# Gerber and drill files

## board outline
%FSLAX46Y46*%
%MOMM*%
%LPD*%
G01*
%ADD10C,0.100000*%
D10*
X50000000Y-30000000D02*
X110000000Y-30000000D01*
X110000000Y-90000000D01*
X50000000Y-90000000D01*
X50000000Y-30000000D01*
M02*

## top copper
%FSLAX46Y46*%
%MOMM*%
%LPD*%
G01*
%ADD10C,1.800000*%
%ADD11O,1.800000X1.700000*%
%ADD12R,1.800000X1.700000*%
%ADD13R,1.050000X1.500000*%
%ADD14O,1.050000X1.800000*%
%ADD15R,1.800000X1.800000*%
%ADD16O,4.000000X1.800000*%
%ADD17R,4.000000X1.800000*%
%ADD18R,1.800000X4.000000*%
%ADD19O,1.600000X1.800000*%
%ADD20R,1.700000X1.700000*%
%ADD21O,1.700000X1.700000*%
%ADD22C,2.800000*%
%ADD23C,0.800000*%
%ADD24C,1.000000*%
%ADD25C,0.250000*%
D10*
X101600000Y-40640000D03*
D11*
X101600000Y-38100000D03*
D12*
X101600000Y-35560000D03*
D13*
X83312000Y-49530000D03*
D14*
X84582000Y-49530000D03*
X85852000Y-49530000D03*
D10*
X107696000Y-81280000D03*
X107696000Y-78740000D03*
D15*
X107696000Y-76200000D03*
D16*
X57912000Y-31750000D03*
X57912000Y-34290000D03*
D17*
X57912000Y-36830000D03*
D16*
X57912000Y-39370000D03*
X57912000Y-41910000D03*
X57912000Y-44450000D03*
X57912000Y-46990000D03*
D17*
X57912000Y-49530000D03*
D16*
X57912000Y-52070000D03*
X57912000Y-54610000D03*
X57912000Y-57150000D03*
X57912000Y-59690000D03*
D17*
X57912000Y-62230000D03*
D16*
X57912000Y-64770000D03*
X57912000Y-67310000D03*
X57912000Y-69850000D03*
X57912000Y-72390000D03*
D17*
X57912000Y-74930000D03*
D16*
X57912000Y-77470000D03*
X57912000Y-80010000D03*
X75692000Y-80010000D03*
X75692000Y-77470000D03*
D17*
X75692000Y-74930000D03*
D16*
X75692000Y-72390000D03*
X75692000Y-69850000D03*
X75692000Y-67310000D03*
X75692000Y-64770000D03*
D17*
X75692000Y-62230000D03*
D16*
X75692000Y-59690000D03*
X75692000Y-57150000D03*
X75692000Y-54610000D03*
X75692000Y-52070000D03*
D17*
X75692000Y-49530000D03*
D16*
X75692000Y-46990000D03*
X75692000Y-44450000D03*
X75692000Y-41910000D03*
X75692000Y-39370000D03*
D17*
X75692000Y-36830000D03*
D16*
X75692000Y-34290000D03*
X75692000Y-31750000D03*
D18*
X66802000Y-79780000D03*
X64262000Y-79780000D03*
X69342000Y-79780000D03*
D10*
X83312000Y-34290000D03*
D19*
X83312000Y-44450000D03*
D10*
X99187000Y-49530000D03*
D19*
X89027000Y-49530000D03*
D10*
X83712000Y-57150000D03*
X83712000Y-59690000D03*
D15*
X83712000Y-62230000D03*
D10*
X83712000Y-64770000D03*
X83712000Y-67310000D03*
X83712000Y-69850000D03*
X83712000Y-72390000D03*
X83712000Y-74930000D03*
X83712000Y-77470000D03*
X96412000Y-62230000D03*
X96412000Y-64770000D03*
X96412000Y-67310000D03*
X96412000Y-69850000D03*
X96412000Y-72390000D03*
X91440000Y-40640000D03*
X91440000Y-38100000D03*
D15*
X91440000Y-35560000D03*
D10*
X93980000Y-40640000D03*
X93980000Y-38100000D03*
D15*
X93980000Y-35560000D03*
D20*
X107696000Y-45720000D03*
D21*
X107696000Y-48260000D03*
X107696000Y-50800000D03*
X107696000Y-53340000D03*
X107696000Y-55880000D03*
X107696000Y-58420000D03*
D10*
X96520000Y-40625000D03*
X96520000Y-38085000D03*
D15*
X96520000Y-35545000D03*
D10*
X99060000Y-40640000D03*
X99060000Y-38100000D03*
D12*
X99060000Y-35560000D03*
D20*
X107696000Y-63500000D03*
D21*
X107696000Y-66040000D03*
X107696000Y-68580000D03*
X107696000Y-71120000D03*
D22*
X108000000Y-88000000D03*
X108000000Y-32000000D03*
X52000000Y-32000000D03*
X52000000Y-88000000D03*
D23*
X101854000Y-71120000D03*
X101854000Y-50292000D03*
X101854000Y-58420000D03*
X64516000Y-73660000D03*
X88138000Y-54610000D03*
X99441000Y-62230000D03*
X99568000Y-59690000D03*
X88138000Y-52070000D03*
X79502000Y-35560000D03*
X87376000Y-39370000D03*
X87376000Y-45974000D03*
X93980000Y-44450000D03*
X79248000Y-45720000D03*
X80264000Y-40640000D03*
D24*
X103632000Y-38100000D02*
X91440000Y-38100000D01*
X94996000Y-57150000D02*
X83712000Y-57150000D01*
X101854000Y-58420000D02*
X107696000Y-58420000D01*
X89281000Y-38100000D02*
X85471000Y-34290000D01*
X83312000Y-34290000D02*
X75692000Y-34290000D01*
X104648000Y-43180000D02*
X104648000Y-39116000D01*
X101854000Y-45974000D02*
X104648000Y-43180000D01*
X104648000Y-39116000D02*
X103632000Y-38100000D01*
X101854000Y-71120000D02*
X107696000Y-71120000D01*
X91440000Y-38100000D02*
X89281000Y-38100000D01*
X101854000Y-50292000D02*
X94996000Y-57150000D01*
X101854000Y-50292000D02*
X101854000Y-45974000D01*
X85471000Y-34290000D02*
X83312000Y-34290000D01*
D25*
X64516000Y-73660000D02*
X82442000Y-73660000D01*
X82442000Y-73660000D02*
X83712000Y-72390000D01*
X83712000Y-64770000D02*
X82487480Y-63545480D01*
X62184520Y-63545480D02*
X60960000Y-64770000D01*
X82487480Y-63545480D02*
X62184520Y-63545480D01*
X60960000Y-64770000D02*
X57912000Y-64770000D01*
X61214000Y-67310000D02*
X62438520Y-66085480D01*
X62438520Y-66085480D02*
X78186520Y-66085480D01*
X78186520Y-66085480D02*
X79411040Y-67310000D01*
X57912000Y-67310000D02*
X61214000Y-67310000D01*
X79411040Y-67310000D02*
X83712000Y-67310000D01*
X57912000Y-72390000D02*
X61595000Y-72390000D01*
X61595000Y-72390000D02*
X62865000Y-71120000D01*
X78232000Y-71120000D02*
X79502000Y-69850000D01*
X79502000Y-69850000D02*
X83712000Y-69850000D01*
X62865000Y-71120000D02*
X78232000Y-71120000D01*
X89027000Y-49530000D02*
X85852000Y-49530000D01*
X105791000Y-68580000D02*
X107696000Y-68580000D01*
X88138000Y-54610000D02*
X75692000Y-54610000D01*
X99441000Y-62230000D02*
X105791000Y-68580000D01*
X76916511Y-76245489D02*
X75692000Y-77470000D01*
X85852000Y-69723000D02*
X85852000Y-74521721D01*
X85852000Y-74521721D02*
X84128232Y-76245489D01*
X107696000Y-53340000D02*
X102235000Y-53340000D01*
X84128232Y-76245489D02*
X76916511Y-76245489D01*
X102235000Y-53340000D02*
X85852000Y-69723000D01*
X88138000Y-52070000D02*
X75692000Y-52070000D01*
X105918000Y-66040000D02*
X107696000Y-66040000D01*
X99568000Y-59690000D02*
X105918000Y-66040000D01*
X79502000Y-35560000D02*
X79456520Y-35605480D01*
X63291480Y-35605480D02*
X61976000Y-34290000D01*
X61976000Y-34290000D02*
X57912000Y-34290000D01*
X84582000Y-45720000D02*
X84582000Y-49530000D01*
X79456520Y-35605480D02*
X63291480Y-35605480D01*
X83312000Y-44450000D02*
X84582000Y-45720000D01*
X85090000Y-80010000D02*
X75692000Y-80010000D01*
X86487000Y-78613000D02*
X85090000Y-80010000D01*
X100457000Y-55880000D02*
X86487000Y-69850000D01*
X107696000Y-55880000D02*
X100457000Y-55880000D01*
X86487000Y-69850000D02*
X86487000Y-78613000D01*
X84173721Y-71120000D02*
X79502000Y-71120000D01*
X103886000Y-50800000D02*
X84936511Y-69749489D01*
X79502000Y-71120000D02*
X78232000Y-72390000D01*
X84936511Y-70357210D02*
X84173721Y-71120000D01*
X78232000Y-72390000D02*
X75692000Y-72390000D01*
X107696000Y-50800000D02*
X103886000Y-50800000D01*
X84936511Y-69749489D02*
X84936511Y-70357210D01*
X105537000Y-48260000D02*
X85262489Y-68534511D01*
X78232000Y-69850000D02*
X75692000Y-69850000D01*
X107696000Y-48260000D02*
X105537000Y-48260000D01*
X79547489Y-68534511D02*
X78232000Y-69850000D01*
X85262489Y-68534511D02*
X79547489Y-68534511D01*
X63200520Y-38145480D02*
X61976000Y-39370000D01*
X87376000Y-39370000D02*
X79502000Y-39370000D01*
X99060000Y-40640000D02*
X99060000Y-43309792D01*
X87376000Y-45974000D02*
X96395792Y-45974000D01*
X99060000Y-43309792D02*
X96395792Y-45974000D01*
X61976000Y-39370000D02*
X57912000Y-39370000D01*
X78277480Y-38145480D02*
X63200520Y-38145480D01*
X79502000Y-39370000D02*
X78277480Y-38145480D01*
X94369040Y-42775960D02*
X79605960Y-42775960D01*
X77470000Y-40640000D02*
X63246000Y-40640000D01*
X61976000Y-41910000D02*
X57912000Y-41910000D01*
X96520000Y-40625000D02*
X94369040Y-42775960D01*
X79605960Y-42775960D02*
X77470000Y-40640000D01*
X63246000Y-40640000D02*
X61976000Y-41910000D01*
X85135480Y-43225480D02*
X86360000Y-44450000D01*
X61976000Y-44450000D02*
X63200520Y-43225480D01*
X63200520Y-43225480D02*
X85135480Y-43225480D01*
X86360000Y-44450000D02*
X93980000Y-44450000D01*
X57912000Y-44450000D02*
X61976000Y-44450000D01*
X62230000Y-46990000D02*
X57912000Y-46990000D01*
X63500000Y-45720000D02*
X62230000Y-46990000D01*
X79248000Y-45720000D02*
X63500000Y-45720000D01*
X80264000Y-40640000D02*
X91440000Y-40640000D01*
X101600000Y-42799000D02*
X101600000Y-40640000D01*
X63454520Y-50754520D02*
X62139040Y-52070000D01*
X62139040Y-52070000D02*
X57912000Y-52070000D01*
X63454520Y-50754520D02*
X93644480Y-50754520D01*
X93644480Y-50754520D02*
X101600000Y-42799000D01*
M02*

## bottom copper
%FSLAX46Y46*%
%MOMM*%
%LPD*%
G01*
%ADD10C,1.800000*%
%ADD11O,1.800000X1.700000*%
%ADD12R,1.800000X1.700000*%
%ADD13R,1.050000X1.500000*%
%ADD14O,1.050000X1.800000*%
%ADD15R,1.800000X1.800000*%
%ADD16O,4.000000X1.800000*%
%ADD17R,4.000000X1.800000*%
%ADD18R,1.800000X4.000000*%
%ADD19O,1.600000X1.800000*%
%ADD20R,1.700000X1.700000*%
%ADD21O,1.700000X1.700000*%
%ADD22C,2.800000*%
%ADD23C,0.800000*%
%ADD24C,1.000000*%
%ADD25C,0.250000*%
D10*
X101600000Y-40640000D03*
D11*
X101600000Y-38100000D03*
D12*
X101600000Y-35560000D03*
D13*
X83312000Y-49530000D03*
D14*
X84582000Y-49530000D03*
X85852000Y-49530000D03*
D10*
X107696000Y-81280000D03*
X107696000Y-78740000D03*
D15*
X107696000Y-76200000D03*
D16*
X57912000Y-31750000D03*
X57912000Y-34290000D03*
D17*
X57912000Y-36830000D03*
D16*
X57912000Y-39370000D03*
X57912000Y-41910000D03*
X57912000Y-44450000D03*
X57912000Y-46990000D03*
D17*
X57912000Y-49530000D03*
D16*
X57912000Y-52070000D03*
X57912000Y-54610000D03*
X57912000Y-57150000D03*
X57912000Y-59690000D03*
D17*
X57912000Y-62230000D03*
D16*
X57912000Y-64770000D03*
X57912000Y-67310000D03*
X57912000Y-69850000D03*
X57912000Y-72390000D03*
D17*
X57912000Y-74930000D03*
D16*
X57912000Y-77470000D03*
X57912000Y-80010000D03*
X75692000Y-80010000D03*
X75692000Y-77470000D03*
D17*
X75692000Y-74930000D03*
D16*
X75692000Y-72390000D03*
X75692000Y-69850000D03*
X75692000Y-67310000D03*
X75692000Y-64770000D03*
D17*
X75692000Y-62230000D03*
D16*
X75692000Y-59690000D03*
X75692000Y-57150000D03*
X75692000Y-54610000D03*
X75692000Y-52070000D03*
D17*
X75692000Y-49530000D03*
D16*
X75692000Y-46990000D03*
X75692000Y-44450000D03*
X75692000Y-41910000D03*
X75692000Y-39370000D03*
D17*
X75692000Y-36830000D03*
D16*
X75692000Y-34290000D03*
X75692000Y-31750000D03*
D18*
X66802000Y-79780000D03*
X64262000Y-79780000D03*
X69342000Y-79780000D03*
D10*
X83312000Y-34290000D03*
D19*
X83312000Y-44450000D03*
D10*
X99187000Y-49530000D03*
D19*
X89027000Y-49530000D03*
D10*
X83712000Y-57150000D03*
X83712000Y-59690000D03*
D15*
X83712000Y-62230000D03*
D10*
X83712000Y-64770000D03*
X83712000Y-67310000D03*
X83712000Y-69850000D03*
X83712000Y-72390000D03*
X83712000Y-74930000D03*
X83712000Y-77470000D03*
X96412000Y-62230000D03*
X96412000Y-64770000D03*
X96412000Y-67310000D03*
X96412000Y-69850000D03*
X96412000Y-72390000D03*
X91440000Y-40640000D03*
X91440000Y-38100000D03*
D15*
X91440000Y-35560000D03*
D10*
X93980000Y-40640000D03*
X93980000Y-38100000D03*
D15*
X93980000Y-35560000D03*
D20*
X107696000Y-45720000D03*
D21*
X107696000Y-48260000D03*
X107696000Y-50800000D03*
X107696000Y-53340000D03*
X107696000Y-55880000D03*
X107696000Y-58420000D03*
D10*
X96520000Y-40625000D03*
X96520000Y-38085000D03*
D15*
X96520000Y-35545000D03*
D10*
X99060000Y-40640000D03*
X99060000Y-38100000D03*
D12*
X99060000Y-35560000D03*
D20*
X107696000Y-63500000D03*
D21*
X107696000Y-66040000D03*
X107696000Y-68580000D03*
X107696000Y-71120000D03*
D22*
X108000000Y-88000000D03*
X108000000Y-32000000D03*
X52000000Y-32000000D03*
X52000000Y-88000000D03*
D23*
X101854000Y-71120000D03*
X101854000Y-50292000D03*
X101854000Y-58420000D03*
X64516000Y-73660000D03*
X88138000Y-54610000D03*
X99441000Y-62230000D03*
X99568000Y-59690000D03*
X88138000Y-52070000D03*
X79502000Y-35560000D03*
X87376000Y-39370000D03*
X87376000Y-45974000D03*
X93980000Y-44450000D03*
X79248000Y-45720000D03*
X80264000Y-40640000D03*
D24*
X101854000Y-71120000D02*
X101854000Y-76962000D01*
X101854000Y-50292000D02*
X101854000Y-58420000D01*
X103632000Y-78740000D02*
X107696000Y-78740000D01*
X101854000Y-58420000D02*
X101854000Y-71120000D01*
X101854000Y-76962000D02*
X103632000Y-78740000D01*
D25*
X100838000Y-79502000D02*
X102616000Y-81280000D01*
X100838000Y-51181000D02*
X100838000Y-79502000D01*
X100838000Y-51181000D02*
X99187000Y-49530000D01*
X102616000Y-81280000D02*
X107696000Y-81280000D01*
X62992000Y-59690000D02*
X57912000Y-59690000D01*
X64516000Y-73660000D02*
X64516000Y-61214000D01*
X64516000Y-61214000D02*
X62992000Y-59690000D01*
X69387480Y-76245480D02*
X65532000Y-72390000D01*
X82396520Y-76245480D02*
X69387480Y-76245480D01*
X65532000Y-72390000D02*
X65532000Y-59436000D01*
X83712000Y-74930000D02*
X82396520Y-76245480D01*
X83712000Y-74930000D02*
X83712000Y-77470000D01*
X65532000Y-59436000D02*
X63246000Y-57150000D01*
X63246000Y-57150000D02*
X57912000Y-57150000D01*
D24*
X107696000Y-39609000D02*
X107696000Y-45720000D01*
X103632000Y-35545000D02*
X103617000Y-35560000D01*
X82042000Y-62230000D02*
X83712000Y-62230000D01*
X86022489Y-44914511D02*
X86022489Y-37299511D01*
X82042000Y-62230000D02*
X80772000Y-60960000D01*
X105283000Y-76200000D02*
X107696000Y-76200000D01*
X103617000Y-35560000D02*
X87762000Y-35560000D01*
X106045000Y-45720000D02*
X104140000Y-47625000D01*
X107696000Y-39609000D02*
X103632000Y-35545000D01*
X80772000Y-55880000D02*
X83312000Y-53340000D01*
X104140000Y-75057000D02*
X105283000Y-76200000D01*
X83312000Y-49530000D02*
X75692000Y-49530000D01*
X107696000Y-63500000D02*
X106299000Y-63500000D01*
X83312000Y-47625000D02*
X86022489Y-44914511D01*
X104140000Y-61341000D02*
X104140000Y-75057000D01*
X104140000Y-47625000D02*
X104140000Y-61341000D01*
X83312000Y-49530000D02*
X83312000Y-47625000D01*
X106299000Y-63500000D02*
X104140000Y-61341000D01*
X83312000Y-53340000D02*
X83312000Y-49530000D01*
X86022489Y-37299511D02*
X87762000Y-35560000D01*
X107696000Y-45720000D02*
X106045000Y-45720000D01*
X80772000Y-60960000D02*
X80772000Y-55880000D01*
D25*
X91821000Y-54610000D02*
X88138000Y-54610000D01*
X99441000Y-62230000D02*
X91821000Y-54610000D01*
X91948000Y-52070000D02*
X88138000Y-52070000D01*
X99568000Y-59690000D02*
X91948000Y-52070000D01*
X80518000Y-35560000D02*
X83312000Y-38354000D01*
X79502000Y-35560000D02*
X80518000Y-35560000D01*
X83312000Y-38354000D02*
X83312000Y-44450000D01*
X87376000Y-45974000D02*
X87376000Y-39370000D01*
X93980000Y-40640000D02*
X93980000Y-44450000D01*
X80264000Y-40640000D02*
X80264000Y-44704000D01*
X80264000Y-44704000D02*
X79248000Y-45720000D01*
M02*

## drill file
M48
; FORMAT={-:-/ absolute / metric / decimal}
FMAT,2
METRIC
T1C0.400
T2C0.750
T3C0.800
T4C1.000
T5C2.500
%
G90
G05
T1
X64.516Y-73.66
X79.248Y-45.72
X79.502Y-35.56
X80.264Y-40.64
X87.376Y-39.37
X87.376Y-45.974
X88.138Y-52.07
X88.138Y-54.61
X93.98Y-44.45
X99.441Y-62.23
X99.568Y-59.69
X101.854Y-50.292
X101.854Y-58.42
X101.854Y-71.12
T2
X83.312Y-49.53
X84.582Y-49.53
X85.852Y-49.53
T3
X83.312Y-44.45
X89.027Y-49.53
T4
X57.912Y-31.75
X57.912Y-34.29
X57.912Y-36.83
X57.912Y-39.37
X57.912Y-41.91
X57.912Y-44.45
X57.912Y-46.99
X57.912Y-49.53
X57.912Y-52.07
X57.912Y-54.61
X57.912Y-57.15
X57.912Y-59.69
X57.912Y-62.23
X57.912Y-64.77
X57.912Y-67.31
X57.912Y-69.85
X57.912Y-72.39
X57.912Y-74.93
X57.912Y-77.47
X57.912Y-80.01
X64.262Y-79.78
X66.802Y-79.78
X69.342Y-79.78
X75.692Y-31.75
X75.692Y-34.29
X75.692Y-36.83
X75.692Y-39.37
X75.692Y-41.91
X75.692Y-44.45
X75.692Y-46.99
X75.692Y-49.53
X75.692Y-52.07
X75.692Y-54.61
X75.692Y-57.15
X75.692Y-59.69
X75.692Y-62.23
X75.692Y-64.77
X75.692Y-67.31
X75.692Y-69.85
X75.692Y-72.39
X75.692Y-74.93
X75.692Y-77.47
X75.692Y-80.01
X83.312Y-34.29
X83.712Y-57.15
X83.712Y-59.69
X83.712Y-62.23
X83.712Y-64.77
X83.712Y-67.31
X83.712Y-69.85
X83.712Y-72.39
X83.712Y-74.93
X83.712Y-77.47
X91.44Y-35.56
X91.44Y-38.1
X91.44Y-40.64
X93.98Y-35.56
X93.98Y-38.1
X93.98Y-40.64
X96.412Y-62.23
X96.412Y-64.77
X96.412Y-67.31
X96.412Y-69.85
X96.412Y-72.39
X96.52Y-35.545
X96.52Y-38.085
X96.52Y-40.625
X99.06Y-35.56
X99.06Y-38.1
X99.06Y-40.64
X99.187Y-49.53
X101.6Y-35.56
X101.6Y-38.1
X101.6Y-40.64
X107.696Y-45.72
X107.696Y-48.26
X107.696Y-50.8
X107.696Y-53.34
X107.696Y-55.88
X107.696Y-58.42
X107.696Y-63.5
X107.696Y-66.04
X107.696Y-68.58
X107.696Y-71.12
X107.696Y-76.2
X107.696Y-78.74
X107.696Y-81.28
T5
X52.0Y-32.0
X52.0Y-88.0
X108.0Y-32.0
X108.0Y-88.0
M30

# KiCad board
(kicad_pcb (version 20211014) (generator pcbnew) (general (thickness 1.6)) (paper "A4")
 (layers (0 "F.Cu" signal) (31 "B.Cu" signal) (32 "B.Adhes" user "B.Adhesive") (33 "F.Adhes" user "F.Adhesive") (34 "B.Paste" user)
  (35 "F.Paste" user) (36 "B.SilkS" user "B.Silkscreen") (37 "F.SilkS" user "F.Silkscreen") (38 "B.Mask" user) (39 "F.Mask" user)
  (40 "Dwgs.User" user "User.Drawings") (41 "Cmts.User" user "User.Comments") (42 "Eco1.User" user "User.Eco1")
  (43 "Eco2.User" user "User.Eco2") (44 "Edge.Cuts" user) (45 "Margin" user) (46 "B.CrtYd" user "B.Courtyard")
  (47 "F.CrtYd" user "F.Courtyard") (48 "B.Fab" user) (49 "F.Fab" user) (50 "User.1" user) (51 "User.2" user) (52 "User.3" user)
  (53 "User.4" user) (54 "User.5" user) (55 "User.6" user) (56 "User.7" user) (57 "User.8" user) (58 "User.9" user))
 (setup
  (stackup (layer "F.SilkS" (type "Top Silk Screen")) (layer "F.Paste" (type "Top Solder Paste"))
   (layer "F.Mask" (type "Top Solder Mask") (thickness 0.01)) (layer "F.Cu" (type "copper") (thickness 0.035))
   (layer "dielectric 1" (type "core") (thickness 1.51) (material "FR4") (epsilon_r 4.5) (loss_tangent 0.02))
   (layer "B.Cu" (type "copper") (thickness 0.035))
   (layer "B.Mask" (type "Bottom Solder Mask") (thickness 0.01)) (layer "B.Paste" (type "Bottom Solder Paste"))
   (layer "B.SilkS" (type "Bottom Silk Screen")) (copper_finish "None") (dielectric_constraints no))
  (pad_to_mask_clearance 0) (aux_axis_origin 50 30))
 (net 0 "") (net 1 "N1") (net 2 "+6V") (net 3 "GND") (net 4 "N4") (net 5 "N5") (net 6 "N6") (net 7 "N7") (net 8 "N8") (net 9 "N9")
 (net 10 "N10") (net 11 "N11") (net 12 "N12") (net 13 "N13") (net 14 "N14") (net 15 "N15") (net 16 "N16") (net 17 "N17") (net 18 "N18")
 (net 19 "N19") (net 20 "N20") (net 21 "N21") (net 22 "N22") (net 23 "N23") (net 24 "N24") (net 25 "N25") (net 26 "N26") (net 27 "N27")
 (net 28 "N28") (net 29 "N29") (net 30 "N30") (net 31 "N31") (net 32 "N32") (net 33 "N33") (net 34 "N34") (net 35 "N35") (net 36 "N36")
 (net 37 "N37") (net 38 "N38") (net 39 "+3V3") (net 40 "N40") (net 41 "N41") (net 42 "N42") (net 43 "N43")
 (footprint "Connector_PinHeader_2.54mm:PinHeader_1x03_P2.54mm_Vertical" (layer "F.Cu") (at 101.6 40.64 180)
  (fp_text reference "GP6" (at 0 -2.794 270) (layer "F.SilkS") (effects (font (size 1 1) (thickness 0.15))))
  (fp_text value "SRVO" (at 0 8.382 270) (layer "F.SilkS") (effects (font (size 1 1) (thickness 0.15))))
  (pad "1" thru_hole circle (at 0 0 180) (size 1.8 1.8) (drill 1) (layers *.Cu *.Mask) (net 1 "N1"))
  (pad "2" thru_hole oval (at 0 2.54 180) (size 1.8 1.7) (drill 1) (layers *.Cu *.Mask) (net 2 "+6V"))
  (pad "3" thru_hole rect (at 0 5.08 180) (size 1.8 1.7) (drill 1) (layers *.Cu *.Mask) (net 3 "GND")))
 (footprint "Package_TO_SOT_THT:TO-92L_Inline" (layer "F.Cu") (at 83.312 49.53)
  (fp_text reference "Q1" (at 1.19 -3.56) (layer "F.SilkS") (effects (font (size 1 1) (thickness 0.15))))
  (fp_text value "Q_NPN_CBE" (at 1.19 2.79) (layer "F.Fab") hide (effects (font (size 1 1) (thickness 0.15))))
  (pad "1" thru_hole rect (at 0 0) (size 1.05 1.5) (drill 0.75) (layers *.Cu *.Mask) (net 3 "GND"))
  (pad "2" thru_hole oval (at 1.27 0) (size 1.05 1.8) (drill 0.75) (layers *.Cu *.Mask) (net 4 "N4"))
  (pad "3" thru_hole oval (at 2.54 0) (size 1.05 1.8) (drill 0.75) (layers *.Cu *.Mask) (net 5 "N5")))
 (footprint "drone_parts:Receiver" (layer "F.Cu") (at 102.616 81.28 90)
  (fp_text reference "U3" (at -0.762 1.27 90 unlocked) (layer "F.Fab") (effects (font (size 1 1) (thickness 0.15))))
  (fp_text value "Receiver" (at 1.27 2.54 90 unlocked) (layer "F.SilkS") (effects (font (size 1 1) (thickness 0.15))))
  (pad "1" thru_hole circle (at 0 5.08 90) (size 1.8 1.8) (drill 1) (layers *.Cu *.Mask) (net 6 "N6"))
  (pad "2" thru_hole circle (at 2.54 5.08 90) (size 1.8 1.8) (drill 1) (layers *.Cu *.Mask) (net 2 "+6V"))
  (pad "3" thru_hole rect (at 5.08 5.08 90) (size 1.8 1.8) (drill 1) (layers *.Cu *.Mask) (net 3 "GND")))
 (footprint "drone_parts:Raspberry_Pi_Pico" (layer "F.Cu") (at 57.912 31.75)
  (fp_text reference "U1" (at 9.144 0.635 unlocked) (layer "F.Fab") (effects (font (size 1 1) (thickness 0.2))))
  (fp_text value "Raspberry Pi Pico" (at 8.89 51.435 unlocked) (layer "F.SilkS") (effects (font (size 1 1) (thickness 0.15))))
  (pad "1" thru_hole oval (at 0 0) (size 4 1.8) (drill 1) (layers *.Cu *.Mask) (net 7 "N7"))
  (pad "2" thru_hole oval (at 0 2.54) (size 4 1.8) (drill 1) (layers *.Cu *.Mask) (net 4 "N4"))
  (pad "3" thru_hole rect (at 0 5.08) (size 4 1.8) (drill 1) (layers *.Cu *.Mask) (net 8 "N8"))
  (pad "4" thru_hole oval (at 0 7.62) (size 4 1.8) (drill 1) (layers *.Cu *.Mask) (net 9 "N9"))
  (pad "5" thru_hole oval (at 0 10.16) (size 4 1.8) (drill 1) (layers *.Cu *.Mask) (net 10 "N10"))
  (pad "6" thru_hole oval (at 0 12.7) (size 4 1.8) (drill 1) (layers *.Cu *.Mask) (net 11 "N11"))
  (pad "7" thru_hole oval (at 0 15.24) (size 4 1.8) (drill 1) (layers *.Cu *.Mask) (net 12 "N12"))
  (pad "8" thru_hole rect (at 0 17.78) (size 4 1.8) (drill 1) (layers *.Cu *.Mask) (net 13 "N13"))
  (pad "9" thru_hole oval (at 0 20.32) (size 4 1.8) (drill 1) (layers *.Cu *.Mask) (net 1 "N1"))
  (pad "10" thru_hole oval (at 0 22.86) (size 4 1.8) (drill 1) (layers *.Cu *.Mask) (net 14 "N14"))
  (pad "11" thru_hole oval (at 0 25.4) (size 4 1.8) (drill 1) (layers *.Cu *.Mask) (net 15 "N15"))
  (pad "12" thru_hole oval (at 0 27.94) (size 4 1.8) (drill 1) (layers *.Cu *.Mask) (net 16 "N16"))
  (pad "13" thru_hole rect (at 0 30.48) (size 4 1.8) (drill 1) (layers *.Cu *.Mask) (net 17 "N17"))
  (pad "14" thru_hole oval (at 0 33.02) (size 4 1.8) (drill 1) (layers *.Cu *.Mask) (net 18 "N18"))
  (pad "15" thru_hole oval (at 0 35.56) (size 4 1.8) (drill 1) (layers *.Cu *.Mask) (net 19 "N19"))
  (pad "16" thru_hole oval (at 0 38.1) (size 4 1.8) (drill 1) (layers *.Cu *.Mask) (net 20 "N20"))
  (pad "17" thru_hole oval (at 0 40.64) (size 4 1.8) (drill 1) (layers *.Cu *.Mask) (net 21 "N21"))
  (pad "18" thru_hole rect (at 0 43.18) (size 4 1.8) (drill 1) (layers *.Cu *.Mask) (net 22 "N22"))
  (pad "19" thru_hole oval (at 0 45.72) (size 4 1.8) (drill 1) (layers *.Cu *.Mask) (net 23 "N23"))
  (pad "20" thru_hole oval (at 0 48.26) (size 4 1.8) (drill 1) (layers *.Cu *.Mask) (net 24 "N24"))
  (pad "21" thru_hole oval (at 17.78 48.26) (size 4 1.8) (drill 1) (layers *.Cu *.Mask) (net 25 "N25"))
  (pad "22" thru_hole oval (at 17.78 45.72) (size 4 1.8) (drill 1) (layers *.Cu *.Mask) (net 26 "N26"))
  (pad "23" thru_hole rect (at 17.78 43.18) (size 4 1.8) (drill 1) (layers *.Cu *.Mask) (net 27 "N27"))
  (pad "24" thru_hole oval (at 17.78 40.64) (size 4 1.8) (drill 1) (layers *.Cu *.Mask) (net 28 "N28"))
  (pad "25" thru_hole oval (at 17.78 38.1) (size 4 1.8) (drill 1) (layers *.Cu *.Mask) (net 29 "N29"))
  (pad "26" thru_hole oval (at 17.78 35.56) (size 4 1.8) (drill 1) (layers *.Cu *.Mask) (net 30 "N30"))
  (pad "27" thru_hole oval (at 17.78 33.02) (size 4 1.8) (drill 1) (layers *.Cu *.Mask) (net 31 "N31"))
  (pad "28" thru_hole rect (at 17.78 30.48) (size 4 1.8) (drill 1) (layers *.Cu *.Mask) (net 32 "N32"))
  (pad "29" thru_hole oval (at 17.78 27.94) (size 4 1.8) (drill 1) (layers *.Cu *.Mask) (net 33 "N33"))
  (pad "30" thru_hole oval (at 17.78 25.4) (size 4 1.8) (drill 1) (layers *.Cu *.Mask) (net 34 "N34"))
  (pad "31" thru_hole oval (at 17.78 22.86) (size 4 1.8) (drill 1) (layers *.Cu *.Mask) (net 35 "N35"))
  (pad "32" thru_hole oval (at 17.78 20.32) (size 4 1.8) (drill 1) (layers *.Cu *.Mask) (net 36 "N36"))
  (pad "33" thru_hole rect (at 17.78 17.78) (size 4 1.8) (drill 1) (layers *.Cu *.Mask) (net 3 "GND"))
  (pad "34" thru_hole oval (at 17.78 15.24) (size 4 1.8) (drill 1) (layers *.Cu *.Mask) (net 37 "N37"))
  (pad "35" thru_hole oval (at 17.78 12.7) (size 4 1.8) (drill 1) (layers *.Cu *.Mask) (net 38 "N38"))
  (pad "36" thru_hole oval (at 17.78 10.16) (size 4 1.8) (drill 1) (layers *.Cu *.Mask) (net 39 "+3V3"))
  (pad "37" thru_hole oval (at 17.78 7.62) (size 4 1.8) (drill 1) (layers *.Cu *.Mask) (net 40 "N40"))
  (pad "38" thru_hole rect (at 17.78 5.08) (size 4 1.8) (drill 1) (layers *.Cu *.Mask) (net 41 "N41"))
  (pad "39" thru_hole oval (at 17.78 2.54) (size 4 1.8) (drill 1) (layers *.Cu *.Mask) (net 2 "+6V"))
  (pad "40" thru_hole oval (at 17.78 0) (size 4 1.8) (drill 1) (layers *.Cu *.Mask) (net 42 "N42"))
  (pad "41" thru_hole rect (at 8.89 48.03) (size 1.8 4) (drill 1) (layers *.Cu *.Mask))
  (pad "42" thru_hole rect (at 6.35 48.03) (size 1.8 4) (drill 1) (layers *.Cu *.Mask))
  (pad "43" thru_hole rect (at 11.43 48.03) (size 1.8 4) (drill 1) (layers *.Cu *.Mask)))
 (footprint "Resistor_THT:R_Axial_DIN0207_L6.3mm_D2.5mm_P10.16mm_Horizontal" (layer "F.Cu") (at 83.312 34.29 -90)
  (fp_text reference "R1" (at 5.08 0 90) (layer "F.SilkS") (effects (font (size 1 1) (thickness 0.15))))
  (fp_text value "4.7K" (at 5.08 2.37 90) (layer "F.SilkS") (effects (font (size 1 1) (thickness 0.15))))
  (pad "1" thru_hole circle (at 0 0 270) (size 1.8 1.8) (drill 1) (layers *.Cu *.Mask) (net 2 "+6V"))
  (pad "2" thru_hole oval (at 10.16 0 270) (size 1.8 1.6) (drill 0.8) (layers *.Cu *.Mask) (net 4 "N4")))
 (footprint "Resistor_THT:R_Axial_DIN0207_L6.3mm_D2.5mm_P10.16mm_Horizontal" (layer "F.Cu") (at 99.187 49.53 180)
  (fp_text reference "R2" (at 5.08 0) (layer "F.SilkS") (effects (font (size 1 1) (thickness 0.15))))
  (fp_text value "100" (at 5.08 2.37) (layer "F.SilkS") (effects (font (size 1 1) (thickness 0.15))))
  (pad "1" thru_hole circle (at 0 0 180) (size 1.8 1.8) (drill 1) (layers *.Cu *.Mask) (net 6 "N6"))
  (pad "2" thru_hole oval (at 10.16 0 180) (size 1.6 1.8) (drill 0.8) (layers *.Cu *.Mask) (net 5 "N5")))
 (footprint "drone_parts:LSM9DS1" (layer "F.Cu") (at 83.712 55.88)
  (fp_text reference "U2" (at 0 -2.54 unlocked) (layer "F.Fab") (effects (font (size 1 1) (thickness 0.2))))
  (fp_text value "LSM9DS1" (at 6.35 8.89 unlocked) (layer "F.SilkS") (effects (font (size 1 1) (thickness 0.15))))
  (pad "1" thru_hole circle (at 0 1.27) (size 1.8 1.8) (drill 1) (layers *.Cu *.Mask) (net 2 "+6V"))
  (pad "2" thru_hole circle (at 0 3.81) (size 1.8 1.8) (drill 1) (layers *.Cu *.Mask) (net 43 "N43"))
  (pad "3" thru_hole rect (at 0 6.35) (size 1.8 1.8) (drill 1) (layers *.Cu *.Mask) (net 3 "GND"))
  (pad "4" thru_hole circle (at 0 8.89) (size 1.8 1.8) (drill 1) (layers *.Cu *.Mask) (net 18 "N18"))
  (pad "5" thru_hole circle (at 0 11.43) (size 1.8 1.8) (drill 1) (layers *.Cu *.Mask) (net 19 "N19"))
  (pad "6" thru_hole circle (at 0 13.97) (size 1.8 1.8) (drill 1) (layers *.Cu *.Mask) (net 21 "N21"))
  (pad "7" thru_hole circle (at 0 16.51) (size 1.8 1.8) (drill 1) (layers *.Cu *.Mask) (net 16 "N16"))
  (pad "8" thru_hole circle (at 0 19.05) (size 1.8 1.8) (drill 1) (layers *.Cu *.Mask) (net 15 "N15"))
  (pad "9" thru_hole circle (at 0 21.59) (size 1.8 1.8) (drill 1) (layers *.Cu *.Mask) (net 15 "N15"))
  (pad "18" thru_hole circle (at 12.7 6.35) (size 1.8 1.8) (drill 1) (layers *.Cu *.Mask))
  (pad "19" thru_hole circle (at 12.7 8.89) (size 1.8 1.8) (drill 1) (layers *.Cu *.Mask))
  (pad "20" thru_hole circle (at 12.7 11.43) (size 1.8 1.8) (drill 1) (layers *.Cu *.Mask))
  (pad "21" thru_hole circle (at 12.7 13.97) (size 1.8 1.8) (drill 1) (layers *.Cu *.Mask))
  (pad "22" thru_hole circle (at 12.7 16.51) (size 1.8 1.8) (drill 1) (layers *.Cu *.Mask)))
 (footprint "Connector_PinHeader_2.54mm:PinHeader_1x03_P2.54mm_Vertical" (layer "F.Cu") (at 91.44 40.64 180)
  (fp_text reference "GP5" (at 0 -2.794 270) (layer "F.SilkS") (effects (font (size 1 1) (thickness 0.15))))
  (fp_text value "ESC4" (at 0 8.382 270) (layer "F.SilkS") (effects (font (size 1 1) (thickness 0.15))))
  (pad "1" thru_hole circle (at 0 0 180) (size 1.8 1.8) (drill 1) (layers *.Cu *.Mask) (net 12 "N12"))
  (pad "2" thru_hole circle (at 0 2.54 180) (size 1.8 1.8) (drill 1) (layers *.Cu *.Mask) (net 2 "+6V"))
  (pad "3" thru_hole rect (at 0 5.08 180) (size 1.8 1.8) (drill 1) (layers *.Cu *.Mask) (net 3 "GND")))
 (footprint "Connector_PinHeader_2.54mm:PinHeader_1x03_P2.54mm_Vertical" (layer "F.Cu") (at 93.98 40.64 180)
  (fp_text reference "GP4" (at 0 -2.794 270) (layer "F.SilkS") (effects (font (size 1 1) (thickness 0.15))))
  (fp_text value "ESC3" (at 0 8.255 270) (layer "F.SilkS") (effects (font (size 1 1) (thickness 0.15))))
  (pad "1" thru_hole circle (at 0 0 180) (size 1.8 1.8) (drill 1) (layers *.Cu *.Mask) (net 11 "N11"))
  (pad "2" thru_hole circle (at 0 2.54 180) (size 1.8 1.8) (drill 1) (layers *.Cu *.Mask) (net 2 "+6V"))
  (pad "3" thru_hole rect (at 0 5.08 180) (size 1.8 1.8) (drill 1) (layers *.Cu *.Mask) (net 3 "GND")))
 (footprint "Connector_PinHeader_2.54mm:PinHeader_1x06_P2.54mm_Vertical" (layer "F.Cu") (at 107.696 45.72)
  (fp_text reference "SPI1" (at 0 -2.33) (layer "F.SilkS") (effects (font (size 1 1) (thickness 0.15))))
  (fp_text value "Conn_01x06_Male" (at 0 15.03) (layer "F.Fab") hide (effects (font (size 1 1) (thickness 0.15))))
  (pad "1" thru_hole rect locked (at 0 0) (size 1.7 1.7) (drill 1) (layers *.Cu *.Mask) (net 3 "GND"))
  (pad "2" thru_hole oval locked (at 0 2.54) (size 1.7 1.7) (drill 1) (layers *.Cu *.Mask) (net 29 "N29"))
  (pad "3" thru_hole oval locked (at 0 5.08) (size 1.7 1.7) (drill 1) (layers *.Cu *.Mask) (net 28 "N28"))
  (pad "4" thru_hole oval locked (at 0 7.62) (size 1.7 1.7) (drill 1) (layers *.Cu *.Mask) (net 26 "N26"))
  (pad "5" thru_hole oval locked (at 0 10.16) (size 1.7 1.7) (drill 1) (layers *.Cu *.Mask) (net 25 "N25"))
  (pad "6" thru_hole oval locked (at 0 12.7) (size 1.7 1.7) (drill 1) (layers *.Cu *.Mask) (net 2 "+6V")))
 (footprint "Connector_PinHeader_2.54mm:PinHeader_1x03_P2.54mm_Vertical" (layer "F.Cu") (at 96.52 40.625 180)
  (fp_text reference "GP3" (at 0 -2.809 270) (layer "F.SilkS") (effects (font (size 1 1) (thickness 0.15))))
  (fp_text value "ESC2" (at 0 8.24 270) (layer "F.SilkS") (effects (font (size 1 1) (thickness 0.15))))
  (pad "1" thru_hole circle (at 0 0 180) (size 1.8 1.8) (drill 1) (layers *.Cu *.Mask) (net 10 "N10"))
  (pad "2" thru_hole circle (at 0 2.54 180) (size 1.8 1.8) (drill 1) (layers *.Cu *.Mask) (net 2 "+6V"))
  (pad "3" thru_hole rect (at 0 5.08 180) (size 1.8 1.8) (drill 1) (layers *.Cu *.Mask) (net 3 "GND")))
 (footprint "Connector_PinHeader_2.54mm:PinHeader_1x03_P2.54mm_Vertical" (layer "F.Cu") (at 99.06 40.64 180)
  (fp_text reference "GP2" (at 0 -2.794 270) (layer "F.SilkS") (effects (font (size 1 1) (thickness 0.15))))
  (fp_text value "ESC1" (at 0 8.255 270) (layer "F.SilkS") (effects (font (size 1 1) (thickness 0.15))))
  (pad "1" thru_hole circle (at 0 0 180) (size 1.8 1.8) (drill 1) (layers *.Cu *.Mask) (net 9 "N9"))
  (pad "2" thru_hole circle (at 0 2.54 180) (size 1.8 1.8) (drill 1) (layers *.Cu *.Mask) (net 2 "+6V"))
  (pad "3" thru_hole rect (at 0 5.08 180) (size 1.8 1.7) (drill 1) (layers *.Cu *.Mask) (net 3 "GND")))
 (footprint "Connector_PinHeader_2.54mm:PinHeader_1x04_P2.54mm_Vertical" (layer "F.Cu") (at 107.696 63.5)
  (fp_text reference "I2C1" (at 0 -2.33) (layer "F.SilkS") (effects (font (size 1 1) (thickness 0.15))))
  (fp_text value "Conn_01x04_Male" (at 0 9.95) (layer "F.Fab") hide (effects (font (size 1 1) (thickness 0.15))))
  (pad "1" thru_hole rect locked (at 0 0) (size 1.7 1.7) (drill 1) (layers *.Cu *.Mask) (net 3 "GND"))
  (pad "2" thru_hole oval locked (at 0 2.54) (size 1.7 1.7) (drill 1) (layers *.Cu *.Mask) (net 36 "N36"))
  (pad "3" thru_hole oval locked (at 0 5.08) (size 1.7 1.7) (drill 1) (layers *.Cu *.Mask) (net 35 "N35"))
  (pad "4" thru_hole oval locked (at 0 7.62) (size 1.7 1.7) (drill 1) (layers *.Cu *.Mask) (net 2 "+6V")))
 (gr_rect (start 50 30) (end 110 90) (layer "Edge.Cuts") (width 0.1) (fill none))
 (via (at 108 88) (size 2.8) (drill 2.5) (layers "F.Cu" "B.Cu") (free) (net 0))
 (via (at 108 32) (size 2.8) (drill 2.5) (layers "F.Cu" "B.Cu") (free) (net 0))
 (via (at 52 32) (size 2.8) (drill 2.5) (layers "F.Cu" "B.Cu") (free) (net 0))
 (via (at 52 88) (size 2.8) (drill 2.5) (layers "F.Cu" "B.Cu") (free) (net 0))
 (segment (start 103.632 38.1) (end 91.44 38.1) (width 1) (layer "F.Cu") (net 2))
 (segment (start 94.996 57.15) (end 83.712 57.15) (width 1) (layer "F.Cu") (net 2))
 (segment (start 101.854 58.42) (end 107.696 58.42) (width 1) (layer "F.Cu") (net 2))
 (segment (start 89.281 38.1) (end 85.471 34.29) (width 1) (layer "F.Cu") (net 2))
 (segment (start 83.312 34.29) (end 75.692 34.29) (width 1) (layer "F.Cu") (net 2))
 (segment (start 104.648 43.18) (end 104.648 39.116) (width 1) (layer "F.Cu") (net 2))
 (segment (start 101.854 45.974) (end 104.648 43.18) (width 1) (layer "F.Cu") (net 2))
 (segment (start 104.648 39.116) (end 103.632 38.1) (width 1) (layer "F.Cu") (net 2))
 (segment (start 101.854 71.12) (end 107.696 71.12) (width 1) (layer "F.Cu") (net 2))
 (segment (start 91.44 38.1) (end 89.281 38.1) (width 1) (layer "F.Cu") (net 2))
 (segment (start 101.854 50.292) (end 94.996 57.15) (width 1) (layer "F.Cu") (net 2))
 (segment (start 101.854 50.292) (end 101.854 45.974) (width 1) (layer "F.Cu") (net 2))
 (segment (start 85.471 34.29) (end 83.312 34.29) (width 1) (layer "F.Cu") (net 2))
 (via (at 101.854 71.12) (size 0.8) (drill 0.4) (layers "F.Cu" "B.Cu") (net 2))
 (via (at 101.854 50.292) (size 0.8) (drill 0.4) (layers "F.Cu" "B.Cu") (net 2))
 (via (at 101.854 58.42) (size 0.8) (drill 0.4) (layers "F.Cu" "B.Cu") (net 2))
 (segment (start 101.854 71.12) (end 101.854 76.962) (width 1) (layer "B.Cu") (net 2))
 (segment (start 101.854 50.292) (end 101.854 58.42) (width 1) (layer "B.Cu") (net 2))
 (segment (start 103.632 78.74) (end 107.696 78.74) (width 1) (layer "B.Cu") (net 2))
 (segment (start 101.854 58.42) (end 101.854 71.12) (width 1) (layer "B.Cu") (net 2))
 (segment (start 101.854 76.962) (end 103.632 78.74) (width 1) (layer "B.Cu") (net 2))
 (segment (start 100.838 79.502) (end 102.616 81.28) (width 0.25) (layer "B.Cu") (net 6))
 (segment (start 100.838 51.181) (end 100.838 79.502) (width 0.25) (layer "B.Cu") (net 6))
 (segment (start 100.838 51.181) (end 99.187 49.53) (width 0.25) (layer "B.Cu") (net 6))
 (segment (start 102.616 81.28) (end 107.696 81.28) (width 0.25) (layer "B.Cu") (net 6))
 (segment (start 64.516 73.66) (end 82.442 73.66) (width 0.25) (layer "F.Cu") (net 16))
 (segment (start 82.442 73.66) (end 83.712 72.39) (width 0.25) (layer "F.Cu") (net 16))
 (via (at 64.516 73.66) (size 0.8) (drill 0.4) (layers "F.Cu" "B.Cu") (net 16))
 (segment (start 62.992 59.69) (end 57.912 59.69) (width 0.25) (layer "B.Cu") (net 16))
 (segment (start 64.516 73.66) (end 64.516 61.214) (width 0.25) (layer "B.Cu") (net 16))
 (segment (start 64.516 61.214) (end 62.992 59.69) (width 0.25) (layer "B.Cu") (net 16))
 (segment (start 83.712 64.77) (end 82.48748 63.54548) (width 0.25) (layer "F.Cu") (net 18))
 (segment (start 62.18452 63.54548) (end 60.96 64.77) (width 0.25) (layer "F.Cu") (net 18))
 (segment (start 82.48748 63.54548) (end 62.18452 63.54548) (width 0.25) (layer "F.Cu") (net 18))
 (segment (start 60.96 64.77) (end 57.912 64.77) (width 0.25) (layer "F.Cu") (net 18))
 (segment (start 61.214 67.31) (end 62.43852 66.08548) (width 0.25) (layer "F.Cu") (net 19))
 (segment (start 62.43852 66.08548) (end 78.18652 66.08548) (width 0.25) (layer "F.Cu") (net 19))
 (segment (start 78.18652 66.08548) (end 79.41104 67.31) (width 0.25) (layer "F.Cu") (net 19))
 (segment (start 57.912 67.31) (end 61.214 67.31) (width 0.25) (layer "F.Cu") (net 19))
 (segment (start 79.41104 67.31) (end 83.712 67.31) (width 0.25) (layer "F.Cu") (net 19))
 (segment (start 57.912 72.39) (end 61.595 72.39) (width 0.25) (layer "F.Cu") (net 21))
 (segment (start 61.595 72.39) (end 62.865 71.12) (width 0.25) (layer "F.Cu") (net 21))
 (segment (start 78.232 71.12) (end 79.502 69.85) (width 0.25) (layer "F.Cu") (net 21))
 (segment (start 79.502 69.85) (end 83.712 69.85) (width 0.25) (layer "F.Cu") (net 21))
 (segment (start 62.865 71.12) (end 78.232 71.12) (width 0.25) (layer "F.Cu") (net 21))
 (segment (start 89.027 49.53) (end 85.852 49.53) (width 0.25) (layer "F.Cu") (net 5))
 (segment (start 69.38748 76.24548) (end 65.532 72.39) (width 0.25) (layer "B.Cu") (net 15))
 (segment (start 82.39652 76.24548) (end 69.38748 76.24548) (width 0.25) (layer "B.Cu") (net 15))
 (segment (start 65.532 72.39) (end 65.532 59.436) (width 0.25) (layer "B.Cu") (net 15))
 (segment (start 83.712 74.93) (end 82.39652 76.24548) (width 0.25) (layer "B.Cu") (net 15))
 (segment (start 83.712 74.93) (end 83.712 77.47) (width 0.25) (layer "B.Cu") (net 15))
 (segment (start 65.532 59.436) (end 63.246 57.15) (width 0.25) (layer "B.Cu") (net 15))
 (segment (start 63.246 57.15) (end 57.912 57.15) (width 0.25) (layer "B.Cu") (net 15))
 (segment (start 107.696 39.609) (end 107.696 45.72) (width 1) (layer "B.Cu") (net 3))
 (segment (start 103.632 35.545) (end 103.617 35.56) (width 1) (layer "B.Cu") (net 3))
 (segment (start 82.042 62.23) (end 83.712 62.23) (width 1) (layer "B.Cu") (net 3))
 (segment (start 86.022489 44.914511) (end 86.022489 37.299511) (width 1) (layer "B.Cu") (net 3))
 (segment (start 82.042 62.23) (end 80.772 60.96) (width 1) (layer "B.Cu") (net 3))
 (segment (start 105.283 76.2) (end 107.696 76.2) (width 1) (layer "B.Cu") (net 3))
 (segment (start 103.617 35.56) (end 87.762 35.56) (width 1) (layer "B.Cu") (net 3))
 (segment (start 106.045 45.72) (end 104.14 47.625) (width 1) (layer "B.Cu") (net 3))
 (segment (start 107.696 39.609) (end 103.632 35.545) (width 1) (layer "B.Cu") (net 3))
 (segment (start 80.772 55.88) (end 83.312 53.34) (width 1) (layer "B.Cu") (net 3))
 (segment (start 104.14 75.057) (end 105.283 76.2) (width 1) (layer "B.Cu") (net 3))
 (segment (start 83.312 49.53) (end 75.692 49.53) (width 1) (layer "B.Cu") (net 3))
 (segment (start 107.696 63.5) (end 106.299 63.5) (width 1) (layer "B.Cu") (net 3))
 (segment (start 83.312 47.625) (end 86.022489 44.914511) (width 1) (layer "B.Cu") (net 3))
 (segment (start 104.14 61.341) (end 104.14 75.057) (width 1) (layer "B.Cu") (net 3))
 (segment (start 104.14 47.625) (end 104.14 61.341) (width 1) (layer "B.Cu") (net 3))
 (segment (start 83.312 49.53) (end 83.312 47.625) (width 1) (layer "B.Cu") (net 3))
 (segment (start 106.299 63.5) (end 104.14 61.341) (width 1) (layer "B.Cu") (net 3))
 (segment (start 83.312 53.34) (end 83.312 49.53) (width 1) (layer "B.Cu") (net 3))
 (segment (start 86.022489 37.299511) (end 87.762 35.56) (width 1) (layer "B.Cu") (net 3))
 (segment (start 107.696 45.72) (end 106.045 45.72) (width 1) (layer "B.Cu") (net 3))
 (segment (start 80.772 60.96) (end 80.772 55.88) (width 1) (layer "B.Cu") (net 3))
 (segment (start 105.791 68.58) (end 107.696 68.58) (width 0.25) (layer "F.Cu") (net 35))
 (segment (start 88.138 54.61) (end 75.692 54.61) (width 0.25) (layer "F.Cu") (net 35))
 (segment (start 99.441 62.23) (end 105.791 68.58) (width 0.25) (layer "F.Cu") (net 35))
 (via (at 88.138 54.61) (size 0.8) (drill 0.4) (layers "F.Cu" "B.Cu") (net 35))
 (via (at 99.441 62.23) (size 0.8) (drill 0.4) (layers "F.Cu" "B.Cu") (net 35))
 (segment (start 91.821 54.61) (end 88.138 54.61) (width 0.25) (layer "B.Cu") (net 35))
 (segment (start 99.441 62.23) (end 91.821 54.61) (width 0.25) (layer "B.Cu") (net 35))
 (segment (start 76.916511 76.245489) (end 75.692 77.47) (width 0.25) (layer "F.Cu") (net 26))
 (segment (start 85.852 69.723) (end 85.852 74.521721) (width 0.25) (layer "F.Cu") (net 26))
 (segment (start 85.852 74.521721) (end 84.128232 76.245489) (width 0.25) (layer "F.Cu") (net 26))
 (segment (start 107.696 53.34) (end 102.235 53.34) (width 0.25) (layer "F.Cu") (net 26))
 (segment (start 84.128232 76.245489) (end 76.916511 76.245489) (width 0.25) (layer "F.Cu") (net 26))
 (segment (start 102.235 53.34) (end 85.852 69.723) (width 0.25) (layer "F.Cu") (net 26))
 (segment (start 88.138 52.07) (end 75.692 52.07) (width 0.25) (layer "F.Cu") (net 36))
 (segment (start 105.918 66.04) (end 107.696 66.04) (width 0.25) (layer "F.Cu") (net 36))
 (segment (start 99.568 59.69) (end 105.918 66.04) (width 0.25) (layer "F.Cu") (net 36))
 (via (at 99.568 59.69) (size 0.8) (drill 0.4) (layers "F.Cu" "B.Cu") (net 36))
 (via (at 88.138 52.07) (size 0.8) (drill 0.4) (layers "F.Cu" "B.Cu") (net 36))
 (segment (start 91.948 52.07) (end 88.138 52.07) (width 0.25) (layer "B.Cu") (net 36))
 (segment (start 99.568 59.69) (end 91.948 52.07) (width 0.25) (layer "B.Cu") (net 36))
 (segment (start 79.502 35.56) (end 79.45652 35.60548) (width 0.25) (layer "F.Cu") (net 4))
 (segment (start 63.29148 35.60548) (end 61.976 34.29) (width 0.25) (layer "F.Cu") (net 4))
 (segment (start 61.976 34.29) (end 57.912 34.29) (width 0.25) (layer "F.Cu") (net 4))
 (segment (start 84.582 45.72) (end 84.582 49.53) (width 0.25) (layer "F.Cu") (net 4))
 (segment (start 79.45652 35.60548) (end 63.29148 35.60548) (width 0.25) (layer "F.Cu") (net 4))
 (segment (start 83.312 44.45) (end 84.582 45.72) (width 0.25) (layer "F.Cu") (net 4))
 (via (at 79.502 35.56) (size 0.8) (drill 0.4) (layers "F.Cu" "B.Cu") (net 4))
 (segment (start 80.518 35.56) (end 83.312 38.354) (width 0.25) (layer "B.Cu") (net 4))
 (segment (start 79.502 35.56) (end 80.518 35.56) (width 0.25) (layer "B.Cu") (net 4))
 (segment (start 83.312 38.354) (end 83.312 44.45) (width 0.25) (layer "B.Cu") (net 4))
 (segment (start 85.09 80.01) (end 75.692 80.01) (width 0.25) (layer "F.Cu") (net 25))
 (segment (start 86.487 78.613) (end 85.09 80.01) (width 0.25) (layer "F.Cu") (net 25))
 (segment (start 100.457 55.88) (end 86.487 69.85) (width 0.25) (layer "F.Cu") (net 25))
 (segment (start 107.696 55.88) (end 100.457 55.88) (width 0.25) (layer "F.Cu") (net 25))
 (segment (start 86.487 69.85) (end 86.487 78.613) (width 0.25) (layer "F.Cu") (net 25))
 (segment (start 84.173721 71.12) (end 79.502 71.12) (width 0.25) (layer "F.Cu") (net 28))
 (segment (start 103.886 50.8) (end 84.936511 69.749489) (width 0.25) (layer "F.Cu") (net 28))
 (segment (start 79.502 71.12) (end 78.232 72.39) (width 0.25) (layer "F.Cu") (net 28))
 (segment (start 84.936511 70.35721) (end 84.173721 71.12) (width 0.25) (layer "F.Cu") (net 28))
 (segment (start 78.232 72.39) (end 75.692 72.39) (width 0.25) (layer "F.Cu") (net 28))
 (segment (start 107.696 50.8) (end 103.886 50.8) (width 0.25) (layer "F.Cu") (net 28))
 (segment (start 84.936511 69.749489) (end 84.936511 70.35721) (width 0.25) (layer "F.Cu") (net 28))
 (segment (start 105.537 48.26) (end 85.262489 68.534511) (width 0.25) (layer "F.Cu") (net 29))
 (segment (start 78.232 69.85) (end 75.692 69.85) (width 0.25) (layer "F.Cu") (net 29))
 (segment (start 107.696 48.26) (end 105.537 48.26) (width 0.25) (layer "F.Cu") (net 29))
 (segment (start 79.547489 68.534511) (end 78.232 69.85) (width 0.25) (layer "F.Cu") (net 29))
 (segment (start 85.262489 68.534511) (end 79.547489 68.534511) (width 0.25) (layer "F.Cu") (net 29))
 (segment (start 63.20052 38.14548) (end 61.976 39.37) (width 0.25) (layer "F.Cu") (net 9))
 (segment (start 87.376 39.37) (end 79.502 39.37) (width 0.25) (layer "F.Cu") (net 9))
 (segment (start 99.06 40.64) (end 99.06 43.309792) (width 0.25) (layer "F.Cu") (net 9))
 (segment (start 87.376 45.974) (end 96.395792 45.974) (width 0.25) (layer "F.Cu") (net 9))
 (segment (start 99.06 43.309792) (end 96.395792 45.974) (width 0.25) (layer "F.Cu") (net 9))
 (segment (start 61.976 39.37) (end 57.912 39.37) (width 0.25) (layer "F.Cu") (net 9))
 (segment (start 78.27748 38.14548) (end 63.20052 38.14548) (width 0.25) (layer "F.Cu") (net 9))
 (segment (start 79.502 39.37) (end 78.27748 38.14548) (width 0.25) (layer "F.Cu") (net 9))
 (via (at 87.376 39.37) (size 0.8) (drill 0.4) (layers "F.Cu" "B.Cu") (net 9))
 (via (at 87.376 45.974) (size 0.8) (drill 0.4) (layers "F.Cu" "B.Cu") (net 9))
 (segment (start 87.376 45.974) (end 87.376 39.37) (width 0.25) (layer "B.Cu") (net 9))
 (segment (start 94.36904 42.77596) (end 79.60596 42.77596) (width 0.25) (layer "F.Cu") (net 10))
 (segment (start 77.47 40.64) (end 63.246 40.64) (width 0.25) (layer "F.Cu") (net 10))
 (segment (start 61.976 41.91) (end 57.912 41.91) (width 0.25) (layer "F.Cu") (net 10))
 (segment (start 96.52 40.625) (end 94.36904 42.77596) (width 0.25) (layer "F.Cu") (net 10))
 (segment (start 79.60596 42.77596) (end 77.47 40.64) (width 0.25) (layer "F.Cu") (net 10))
 (segment (start 63.246 40.64) (end 61.976 41.91) (width 0.25) (layer "F.Cu") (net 10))
 (segment (start 85.13548 43.22548) (end 86.36 44.45) (width 0.25) (layer "F.Cu") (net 11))
 (segment (start 61.976 44.45) (end 63.20052 43.22548) (width 0.25) (layer "F.Cu") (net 11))
 (segment (start 63.20052 43.22548) (end 85.13548 43.22548) (width 0.25) (layer "F.Cu") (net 11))
 (segment (start 86.36 44.45) (end 93.98 44.45) (width 0.25) (layer "F.Cu") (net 11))
 (segment (start 57.912 44.45) (end 61.976 44.45) (width 0.25) (layer "F.Cu") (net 11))
 (via (at 93.98 44.45) (size 0.8) (drill 0.4) (layers "F.Cu" "B.Cu") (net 11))
 (segment (start 93.98 40.64) (end 93.98 44.45) (width 0.25) (layer "B.Cu") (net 11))
 (segment (start 62.23 46.99) (end 57.912 46.99) (width 0.25) (layer "F.Cu") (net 12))
 (segment (start 63.5 45.72) (end 62.23 46.99) (width 0.25) (layer "F.Cu") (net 12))
 (segment (start 79.248 45.72) (end 63.5 45.72) (width 0.25) (layer "F.Cu") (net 12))
 (segment (start 80.264 40.64) (end 91.44 40.64) (width 0.25) (layer "F.Cu") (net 12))
 (via (at 79.248 45.72) (size 0.8) (drill 0.4) (layers "F.Cu" "B.Cu") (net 12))
 (via (at 80.264 40.64) (size 0.8) (drill 0.4) (layers "F.Cu" "B.Cu") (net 12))
 (segment (start 80.264 40.64) (end 80.264 44.704) (width 0.25) (layer "B.Cu") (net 12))
 (segment (start 80.264 44.704) (end 79.248 45.72) (width 0.25) (layer "B.Cu") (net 12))
 (segment (start 101.6 42.799) (end 101.6 40.64) (width 0.25) (layer "F.Cu") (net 1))
 (segment (start 63.45452 50.75452) (end 62.13904 52.07) (width 0.25) (layer "F.Cu") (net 1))
 (segment (start 62.13904 52.07) (end 57.912 52.07) (width 0.25) (layer "F.Cu") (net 1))
 (segment (start 63.45452 50.75452) (end 93.64448 50.75452) (width 0.25) (layer "F.Cu") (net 1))
 (segment (start 93.64448 50.75452) (end 101.6 42.799) (width 0.25) (layer "F.Cu") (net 1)))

